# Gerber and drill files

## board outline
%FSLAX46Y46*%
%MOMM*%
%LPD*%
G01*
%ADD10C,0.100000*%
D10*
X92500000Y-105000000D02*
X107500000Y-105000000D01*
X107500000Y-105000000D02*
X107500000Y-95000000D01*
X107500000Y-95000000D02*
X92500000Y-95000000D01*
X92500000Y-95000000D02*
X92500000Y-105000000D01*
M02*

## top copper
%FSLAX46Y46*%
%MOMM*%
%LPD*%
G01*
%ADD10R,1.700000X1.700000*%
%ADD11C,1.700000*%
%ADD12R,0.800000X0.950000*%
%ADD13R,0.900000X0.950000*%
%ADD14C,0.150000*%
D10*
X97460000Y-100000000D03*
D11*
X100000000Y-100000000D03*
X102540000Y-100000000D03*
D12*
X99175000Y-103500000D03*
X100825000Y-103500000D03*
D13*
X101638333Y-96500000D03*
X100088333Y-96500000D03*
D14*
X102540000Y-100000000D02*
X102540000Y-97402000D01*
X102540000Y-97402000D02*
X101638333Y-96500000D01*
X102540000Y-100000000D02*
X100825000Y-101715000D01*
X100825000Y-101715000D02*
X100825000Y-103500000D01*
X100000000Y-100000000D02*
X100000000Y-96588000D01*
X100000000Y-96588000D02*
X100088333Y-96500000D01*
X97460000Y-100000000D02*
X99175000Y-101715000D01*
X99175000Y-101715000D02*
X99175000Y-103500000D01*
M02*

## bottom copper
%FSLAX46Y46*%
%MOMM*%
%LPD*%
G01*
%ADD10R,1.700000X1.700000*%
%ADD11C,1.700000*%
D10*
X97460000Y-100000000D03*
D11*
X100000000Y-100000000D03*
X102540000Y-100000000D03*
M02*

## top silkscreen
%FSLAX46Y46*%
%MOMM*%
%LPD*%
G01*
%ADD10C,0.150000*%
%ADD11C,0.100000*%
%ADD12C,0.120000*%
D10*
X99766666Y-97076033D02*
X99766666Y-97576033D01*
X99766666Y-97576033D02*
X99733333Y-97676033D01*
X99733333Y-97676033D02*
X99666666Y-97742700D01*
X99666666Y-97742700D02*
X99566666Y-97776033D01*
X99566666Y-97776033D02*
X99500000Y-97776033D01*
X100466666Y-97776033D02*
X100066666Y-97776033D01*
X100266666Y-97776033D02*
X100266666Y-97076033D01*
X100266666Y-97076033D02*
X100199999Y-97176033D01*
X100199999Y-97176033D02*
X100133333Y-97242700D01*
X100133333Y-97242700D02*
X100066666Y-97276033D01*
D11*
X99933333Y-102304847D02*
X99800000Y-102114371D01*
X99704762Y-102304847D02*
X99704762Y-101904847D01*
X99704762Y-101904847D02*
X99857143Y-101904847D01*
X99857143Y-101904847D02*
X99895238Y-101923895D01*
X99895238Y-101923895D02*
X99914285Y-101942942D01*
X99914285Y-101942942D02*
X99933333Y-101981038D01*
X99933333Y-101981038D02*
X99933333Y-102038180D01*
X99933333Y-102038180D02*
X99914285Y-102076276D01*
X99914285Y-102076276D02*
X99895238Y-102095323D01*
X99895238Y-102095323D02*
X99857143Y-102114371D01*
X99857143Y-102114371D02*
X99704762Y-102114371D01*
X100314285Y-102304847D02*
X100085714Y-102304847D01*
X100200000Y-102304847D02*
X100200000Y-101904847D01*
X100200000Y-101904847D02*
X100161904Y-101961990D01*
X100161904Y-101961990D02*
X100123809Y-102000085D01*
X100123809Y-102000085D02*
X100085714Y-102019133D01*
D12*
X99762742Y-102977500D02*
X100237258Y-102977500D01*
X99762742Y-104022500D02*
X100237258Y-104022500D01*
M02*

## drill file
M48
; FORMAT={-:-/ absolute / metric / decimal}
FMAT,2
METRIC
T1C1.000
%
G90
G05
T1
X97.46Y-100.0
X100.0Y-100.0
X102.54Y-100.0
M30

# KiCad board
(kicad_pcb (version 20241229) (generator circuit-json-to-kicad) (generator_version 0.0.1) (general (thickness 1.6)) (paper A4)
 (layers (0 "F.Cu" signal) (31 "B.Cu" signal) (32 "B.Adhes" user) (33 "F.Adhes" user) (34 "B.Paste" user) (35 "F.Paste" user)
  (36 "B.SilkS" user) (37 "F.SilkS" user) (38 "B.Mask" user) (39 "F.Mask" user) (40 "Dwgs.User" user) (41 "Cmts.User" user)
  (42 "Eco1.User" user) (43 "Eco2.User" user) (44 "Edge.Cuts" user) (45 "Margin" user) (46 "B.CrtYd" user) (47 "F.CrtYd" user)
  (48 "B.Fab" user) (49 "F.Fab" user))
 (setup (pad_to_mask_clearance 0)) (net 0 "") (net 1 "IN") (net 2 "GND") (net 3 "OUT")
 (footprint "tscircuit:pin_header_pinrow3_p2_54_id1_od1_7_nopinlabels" (layer F.Cu) (at 100 100 0)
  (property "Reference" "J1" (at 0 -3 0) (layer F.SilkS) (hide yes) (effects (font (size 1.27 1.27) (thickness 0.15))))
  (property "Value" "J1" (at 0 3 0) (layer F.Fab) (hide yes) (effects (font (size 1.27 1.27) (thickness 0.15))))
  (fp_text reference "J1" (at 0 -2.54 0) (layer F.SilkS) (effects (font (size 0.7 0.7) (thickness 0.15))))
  (pad "1" thru_hole rect (at -2.54 0 0) (size 1.7 1.7) (drill 1) (layers *.Cu *.Mask) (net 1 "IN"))
  (pad "2" thru_hole circle (at 0 0 0) (size 1.7 1.7) (drill 1) (layers *.Cu *.Mask) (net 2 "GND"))
  (pad "3" thru_hole circle (at 2.54 0 0) (size 1.7 1.7) (drill 1) (layers *.Cu *.Mask) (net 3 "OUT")))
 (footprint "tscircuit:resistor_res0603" (layer F.Cu) (at 100 103.5 0)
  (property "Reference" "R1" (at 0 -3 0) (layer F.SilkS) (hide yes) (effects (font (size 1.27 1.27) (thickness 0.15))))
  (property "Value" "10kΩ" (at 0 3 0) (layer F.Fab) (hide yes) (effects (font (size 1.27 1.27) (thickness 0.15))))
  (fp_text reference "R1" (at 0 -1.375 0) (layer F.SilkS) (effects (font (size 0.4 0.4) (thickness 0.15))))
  (fp_line (start -0.237258 -0.5225) (end 0.237258 -0.5225) (stroke (width 0.12) (type default)) (layer F.SilkS))
  (fp_line (start -0.237258 0.5225) (end 0.237258 0.5225) (stroke (width 0.12) (type default)) (layer F.SilkS))
  (pad "1" smd rect (at -0.825 0 0) (size 0.8 0.95) (layers F.Cu F.Mask) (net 1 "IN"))
  (pad "2" smd rect (at 0.825 0 0) (size 0.8 0.95) (layers F.Cu F.Mask) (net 3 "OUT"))
  (pad "" smd rect (at -0.825 0 0) (size 0.5599999999999999 0.6649999999999999) (layers F.Paste))
  (pad "" smd rect (at 0.825 0 0) (size 0.5599999999999999 0.6649999999999999) (layers F.Paste)))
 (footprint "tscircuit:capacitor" (layer F.Cu) (at 100.86333333333333 96.5 180)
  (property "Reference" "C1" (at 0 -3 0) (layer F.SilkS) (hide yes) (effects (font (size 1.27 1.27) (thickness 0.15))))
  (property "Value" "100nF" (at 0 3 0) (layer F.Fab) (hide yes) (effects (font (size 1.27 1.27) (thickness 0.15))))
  (pad "1" smd rect (at -0.7749999999999999 0 0) (size 0.9 0.95) (layers F.Cu F.Mask) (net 3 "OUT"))
  (pad "2" smd rect (at 0.775 0 0) (size 0.9 0.95) (layers F.Cu F.Mask) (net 2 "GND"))
  (pad "" smd rect (at -0.7749999999999999 0 0) (size 0.63 0.6649999999999999) (layers F.Paste))
  (pad "" smd rect (at 0.775 0 0) (size 0.63 0.6649999999999999) (layers F.Paste)))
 (segment (start 102.54 100) (end 102.54 97.402) (width 0.15) (layer F.Cu) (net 3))
 (segment (start 102.54 97.402) (end 101.63833333333334 96.5) (width 0.15) (layer F.Cu) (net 3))
 (segment (start 102.54 100) (end 100.825 101.715) (width 0.15) (layer F.Cu) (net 3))
 (segment (start 100.825 101.715) (end 100.825 103.5) (width 0.15) (layer F.Cu) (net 3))
 (segment (start 100 100) (end 100 96.588) (width 0.15) (layer F.Cu) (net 2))
 (segment (start 100 96.588) (end 100.08833333333334 96.5) (width 0.15) (layer F.Cu) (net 2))
 (segment (start 97.46 100) (end 99.175 101.715) (width 0.15) (layer F.Cu) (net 1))
 (segment (start 99.175 101.715) (end 99.175 103.5) (width 0.15) (layer F.Cu) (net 1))
 (gr_line (start 92.5 105) (end 107.5 105) (width 0.1) (layer Edge.Cuts))
 (gr_line (start 107.5 105) (end 107.5 95) (width 0.1) (layer Edge.Cuts))
 (gr_line (start 107.5 95) (end 92.5 95) (width 0.1) (layer Edge.Cuts))
 (gr_line (start 92.5 95) (end 92.5 105) (width 0.1) (layer Edge.Cuts)))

